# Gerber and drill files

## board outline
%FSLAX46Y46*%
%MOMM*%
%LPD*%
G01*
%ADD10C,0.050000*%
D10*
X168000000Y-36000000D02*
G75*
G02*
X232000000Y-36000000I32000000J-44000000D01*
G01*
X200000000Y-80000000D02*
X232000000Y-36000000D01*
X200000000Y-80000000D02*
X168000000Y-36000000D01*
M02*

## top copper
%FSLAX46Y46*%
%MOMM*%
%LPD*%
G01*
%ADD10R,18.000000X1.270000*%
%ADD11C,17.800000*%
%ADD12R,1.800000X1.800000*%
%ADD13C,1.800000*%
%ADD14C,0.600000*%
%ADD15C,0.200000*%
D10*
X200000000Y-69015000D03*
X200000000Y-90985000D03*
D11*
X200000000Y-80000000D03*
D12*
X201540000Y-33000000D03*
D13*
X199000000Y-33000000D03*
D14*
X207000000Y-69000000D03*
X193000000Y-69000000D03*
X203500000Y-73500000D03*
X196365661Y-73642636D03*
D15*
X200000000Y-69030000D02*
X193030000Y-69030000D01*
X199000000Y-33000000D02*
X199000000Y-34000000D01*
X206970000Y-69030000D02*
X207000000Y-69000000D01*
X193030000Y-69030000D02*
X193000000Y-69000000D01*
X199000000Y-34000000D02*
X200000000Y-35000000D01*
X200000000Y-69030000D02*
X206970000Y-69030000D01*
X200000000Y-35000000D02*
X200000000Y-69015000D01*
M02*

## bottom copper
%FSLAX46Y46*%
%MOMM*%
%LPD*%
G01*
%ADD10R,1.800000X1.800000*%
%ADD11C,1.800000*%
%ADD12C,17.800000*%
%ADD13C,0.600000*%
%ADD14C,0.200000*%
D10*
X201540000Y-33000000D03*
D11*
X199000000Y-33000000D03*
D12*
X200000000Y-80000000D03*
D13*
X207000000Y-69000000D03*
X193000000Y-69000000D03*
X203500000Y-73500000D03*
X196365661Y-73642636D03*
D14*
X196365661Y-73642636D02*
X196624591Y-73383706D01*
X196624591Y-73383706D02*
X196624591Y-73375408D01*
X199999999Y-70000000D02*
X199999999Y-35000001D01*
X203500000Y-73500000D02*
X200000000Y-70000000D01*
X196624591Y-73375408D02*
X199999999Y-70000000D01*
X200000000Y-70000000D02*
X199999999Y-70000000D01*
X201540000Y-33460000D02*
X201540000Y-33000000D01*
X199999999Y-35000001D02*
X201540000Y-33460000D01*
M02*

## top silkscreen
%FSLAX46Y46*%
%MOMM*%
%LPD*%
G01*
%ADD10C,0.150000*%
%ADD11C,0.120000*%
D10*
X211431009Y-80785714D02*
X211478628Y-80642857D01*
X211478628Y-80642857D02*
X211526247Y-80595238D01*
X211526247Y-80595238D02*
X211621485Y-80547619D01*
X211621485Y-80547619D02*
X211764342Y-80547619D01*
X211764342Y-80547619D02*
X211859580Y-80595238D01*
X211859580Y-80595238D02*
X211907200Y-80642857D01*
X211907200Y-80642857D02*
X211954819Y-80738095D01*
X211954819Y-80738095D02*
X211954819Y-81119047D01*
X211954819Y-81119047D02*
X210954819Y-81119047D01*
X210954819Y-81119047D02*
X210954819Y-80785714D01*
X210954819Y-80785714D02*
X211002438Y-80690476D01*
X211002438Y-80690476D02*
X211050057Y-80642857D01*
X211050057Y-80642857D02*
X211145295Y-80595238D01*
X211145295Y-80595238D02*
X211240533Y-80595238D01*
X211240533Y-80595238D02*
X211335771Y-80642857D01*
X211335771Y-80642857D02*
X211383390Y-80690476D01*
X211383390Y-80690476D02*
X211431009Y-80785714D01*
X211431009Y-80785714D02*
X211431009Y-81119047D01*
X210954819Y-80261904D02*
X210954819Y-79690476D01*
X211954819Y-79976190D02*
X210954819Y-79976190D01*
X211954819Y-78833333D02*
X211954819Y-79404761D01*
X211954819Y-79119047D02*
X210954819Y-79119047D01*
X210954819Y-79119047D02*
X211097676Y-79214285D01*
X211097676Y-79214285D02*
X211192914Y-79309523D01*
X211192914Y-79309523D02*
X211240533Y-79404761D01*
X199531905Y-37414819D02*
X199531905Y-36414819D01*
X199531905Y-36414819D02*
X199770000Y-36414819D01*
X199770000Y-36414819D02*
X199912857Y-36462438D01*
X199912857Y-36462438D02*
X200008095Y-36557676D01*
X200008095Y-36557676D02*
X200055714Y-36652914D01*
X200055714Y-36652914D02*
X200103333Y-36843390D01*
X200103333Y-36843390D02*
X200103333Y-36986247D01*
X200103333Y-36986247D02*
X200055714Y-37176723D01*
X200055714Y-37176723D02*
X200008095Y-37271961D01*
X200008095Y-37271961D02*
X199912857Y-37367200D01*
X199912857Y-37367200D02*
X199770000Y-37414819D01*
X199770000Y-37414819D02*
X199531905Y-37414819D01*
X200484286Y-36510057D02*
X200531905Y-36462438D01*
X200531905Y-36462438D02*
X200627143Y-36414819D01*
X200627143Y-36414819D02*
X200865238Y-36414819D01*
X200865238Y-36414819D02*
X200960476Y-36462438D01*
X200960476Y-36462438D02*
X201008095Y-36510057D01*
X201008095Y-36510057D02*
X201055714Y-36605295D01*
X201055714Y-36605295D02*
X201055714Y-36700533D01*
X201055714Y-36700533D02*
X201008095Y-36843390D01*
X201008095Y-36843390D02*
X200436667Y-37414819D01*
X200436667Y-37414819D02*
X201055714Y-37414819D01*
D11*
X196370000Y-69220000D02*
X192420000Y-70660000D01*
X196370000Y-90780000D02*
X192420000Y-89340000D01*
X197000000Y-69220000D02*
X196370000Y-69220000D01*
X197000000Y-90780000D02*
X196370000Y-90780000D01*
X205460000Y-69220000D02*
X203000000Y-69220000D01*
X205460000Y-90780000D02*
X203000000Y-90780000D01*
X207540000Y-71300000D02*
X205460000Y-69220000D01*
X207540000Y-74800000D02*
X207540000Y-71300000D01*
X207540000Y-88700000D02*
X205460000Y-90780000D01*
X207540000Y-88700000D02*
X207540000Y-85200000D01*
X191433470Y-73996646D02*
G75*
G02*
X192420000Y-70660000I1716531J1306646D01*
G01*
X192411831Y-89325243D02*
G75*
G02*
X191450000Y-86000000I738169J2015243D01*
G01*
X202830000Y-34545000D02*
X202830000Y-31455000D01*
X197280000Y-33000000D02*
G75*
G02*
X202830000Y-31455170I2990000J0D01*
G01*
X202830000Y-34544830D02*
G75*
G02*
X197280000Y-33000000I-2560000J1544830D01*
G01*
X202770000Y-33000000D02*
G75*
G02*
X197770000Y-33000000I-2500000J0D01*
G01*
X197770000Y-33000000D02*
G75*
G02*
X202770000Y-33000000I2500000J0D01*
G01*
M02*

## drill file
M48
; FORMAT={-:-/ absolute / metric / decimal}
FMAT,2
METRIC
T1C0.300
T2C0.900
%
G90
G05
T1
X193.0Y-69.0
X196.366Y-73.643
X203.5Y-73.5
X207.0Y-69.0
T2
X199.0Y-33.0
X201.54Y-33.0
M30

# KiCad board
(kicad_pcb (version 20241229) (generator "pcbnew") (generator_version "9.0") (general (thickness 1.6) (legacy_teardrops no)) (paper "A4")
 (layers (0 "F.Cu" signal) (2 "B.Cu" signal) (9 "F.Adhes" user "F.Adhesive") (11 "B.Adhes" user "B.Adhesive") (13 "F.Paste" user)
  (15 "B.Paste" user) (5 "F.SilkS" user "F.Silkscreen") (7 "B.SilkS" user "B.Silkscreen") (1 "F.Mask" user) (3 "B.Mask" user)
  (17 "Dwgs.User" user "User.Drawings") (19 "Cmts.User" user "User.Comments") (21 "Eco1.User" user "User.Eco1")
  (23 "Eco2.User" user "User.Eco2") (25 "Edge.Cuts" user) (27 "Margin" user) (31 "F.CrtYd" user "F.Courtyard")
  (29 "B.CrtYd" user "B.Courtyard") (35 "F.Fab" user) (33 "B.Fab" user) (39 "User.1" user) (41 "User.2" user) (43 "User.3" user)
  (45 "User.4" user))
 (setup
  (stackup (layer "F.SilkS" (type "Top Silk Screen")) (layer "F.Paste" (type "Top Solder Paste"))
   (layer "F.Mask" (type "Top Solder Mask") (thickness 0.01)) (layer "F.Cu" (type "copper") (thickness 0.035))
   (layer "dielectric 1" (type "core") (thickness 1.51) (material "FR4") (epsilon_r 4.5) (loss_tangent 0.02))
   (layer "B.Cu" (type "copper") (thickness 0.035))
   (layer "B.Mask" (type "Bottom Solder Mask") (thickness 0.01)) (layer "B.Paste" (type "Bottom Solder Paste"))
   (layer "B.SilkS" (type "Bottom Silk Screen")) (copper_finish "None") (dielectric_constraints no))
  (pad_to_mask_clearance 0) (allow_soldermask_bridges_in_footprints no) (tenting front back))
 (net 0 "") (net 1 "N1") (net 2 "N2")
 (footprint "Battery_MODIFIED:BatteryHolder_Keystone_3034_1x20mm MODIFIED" (layer "F.Cu") (at 200 80 -90)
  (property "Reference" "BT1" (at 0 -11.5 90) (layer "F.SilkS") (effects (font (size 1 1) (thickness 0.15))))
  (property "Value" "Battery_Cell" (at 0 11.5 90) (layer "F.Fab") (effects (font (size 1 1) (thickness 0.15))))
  (fp_line (start -10.78 3.63) (end -9.34 7.58) (stroke (width 0.12) (type solid)) (layer "F.SilkS"))
  (fp_line (start 10.78 3.63) (end 9.34 7.58) (stroke (width 0.12) (type solid)) (layer "F.SilkS"))
  (fp_line (start -10.78 3) (end -10.78 3.63) (stroke (width 0.12) (type solid)) (layer "F.SilkS"))
  (fp_line (start 10.78 3) (end 10.78 3.63) (stroke (width 0.12) (type solid)) (layer "F.SilkS"))
  (fp_line (start -10.78 -5.46) (end -10.78 -3) (stroke (width 0.12) (type solid)) (layer "F.SilkS"))
  (fp_line (start 10.78 -5.46) (end 10.78 -3) (stroke (width 0.12) (type solid)) (layer "F.SilkS"))
  (fp_line (start -8.7 -7.54) (end -10.78 -5.46) (stroke (width 0.12) (type solid)) (layer "F.SilkS"))
  (fp_line (start -5.2 -7.54) (end -8.7 -7.54) (stroke (width 0.12) (type solid)) (layer "F.SilkS"))
  (fp_line (start 8.7 -7.54) (end 10.78 -5.46) (stroke (width 0.12) (type solid)) (layer "F.SilkS"))
  (fp_line (start 8.7 -7.54) (end 5.2 -7.54) (stroke (width 0.12) (type solid)) (layer "F.SilkS"))
  (fp_arc (start -6.003354 8.56653) (mid -7.921654 8.918738) (end -9.34 7.58) (stroke (width 0.12) (type solid)) (layer "F.SilkS"))
  (fp_arc (start 9.325243 7.588169) (mid 7.90634 8.911668) (end 6 8.55) (stroke (width 0.12) (type solid)) (layer "F.SilkS"))
  (pad "1" smd rect (at -10.985 0 270) (size 1.27 18) (layers "F.Cu" "F.Mask" "F.Paste") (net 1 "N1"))
  (pad "1" smd rect (at 10.985 0 270) (size 1.27 18) (layers "F.Cu" "F.Mask" "F.Paste") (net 1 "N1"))
  (pad "2" smd circle (at 0 0 270) (size 17.8 17.8) (layers "F.Cu" "F.Mask") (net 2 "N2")))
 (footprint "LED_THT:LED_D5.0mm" (layer "F.Cu") (at 201.54 33 180)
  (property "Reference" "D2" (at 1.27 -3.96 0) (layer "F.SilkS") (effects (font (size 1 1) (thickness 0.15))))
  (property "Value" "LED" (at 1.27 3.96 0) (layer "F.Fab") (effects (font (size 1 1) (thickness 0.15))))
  (fp_line (start -1.29 -1.545) (end -1.29 1.545) (stroke (width 0.12) (type solid)) (layer "F.SilkS"))
  (fp_arc (start 4.26 0) (mid 2.071779 2.880495) (end -1.29 1.54483) (stroke (width 0.12) (type solid)) (layer "F.SilkS"))
  (fp_arc (start -1.29 -1.54483) (mid 2.071779 -2.880495) (end 4.26 0) (stroke (width 0.12) (type solid)) (layer "F.SilkS"))
  (fp_circle (center 1.27 0) (end 3.77 0) (stroke (width 0.12) (type solid)) (fill no) (layer "F.SilkS"))
  (pad "1" thru_hole rect (at 0 0 180) (size 1.8 1.8) (drill 0.9) (layers "*.Cu" "*.Mask") (remove_unused_layers no) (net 2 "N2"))
  (pad "2" thru_hole circle (at 2.54 0 180) (size 1.8 1.8) (drill 0.9) (layers "*.Cu" "*.Mask") (remove_unused_layers no) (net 1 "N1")))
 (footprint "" (layer "B.Cu") (at 200 80 180)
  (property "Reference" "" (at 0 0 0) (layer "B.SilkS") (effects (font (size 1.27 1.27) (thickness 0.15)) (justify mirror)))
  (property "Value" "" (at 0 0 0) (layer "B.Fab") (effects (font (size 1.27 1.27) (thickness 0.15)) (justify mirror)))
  (pad "2" smd circle (at 0 0 90) (size 17.8 17.8) (layers "B.Cu" "B.Mask") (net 2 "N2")))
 (gr_arc (start 168 36) (mid 200 25.594118) (end 232 36) (stroke (width 0.05) (type default)) (layer "Edge.Cuts"))
 (gr_line (start 200 80) (end 232 36) (stroke (width 0.05) (type default)) (layer "Edge.Cuts"))
 (gr_line (start 200 80) (end 168 36) (stroke (width 0.05) (type default)) (layer "Edge.Cuts"))
 (segment (start 200 69.03) (end 193.03 69.03) (width 0.2) (layer "F.Cu") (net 1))
 (segment (start 199 33) (end 199 34) (width 0.2) (layer "F.Cu") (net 1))
 (segment (start 206.97 69.03) (end 207 69) (width 0.2) (layer "F.Cu") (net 1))
 (segment (start 193.03 69.03) (end 193 69) (width 0.2) (layer "F.Cu") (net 1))
 (segment (start 199 34) (end 200 35) (width 0.2) (layer "F.Cu") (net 1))
 (segment (start 200 69.03) (end 206.97 69.03) (width 0.2) (layer "F.Cu") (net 1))
 (segment (start 200 35) (end 200 69.015) (width 0.2) (layer "F.Cu") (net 1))
 (via (at 207 69) (size 0.6) (drill 0.3) (layers "F.Cu" "B.Cu") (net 1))
 (via (at 193 69) (size 0.6) (drill 0.3) (layers "F.Cu" "B.Cu") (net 1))
 (via (at 203.5 73.5) (size 0.6) (drill 0.3) (layers "F.Cu" "B.Cu") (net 2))
 (via (at 196.365661 73.642636) (size 0.6) (drill 0.3) (layers "F.Cu" "B.Cu") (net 2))
 (segment (start 196.365661 73.642636) (end 196.624591 73.383706) (width 0.2) (layer "B.Cu") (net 2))
 (segment (start 196.624591 73.383706) (end 196.624591 73.375408) (width 0.2) (layer "B.Cu") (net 2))
 (segment (start 199.999999 70) (end 199.999999 35.000001) (width 0.2) (layer "B.Cu") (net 2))
 (segment (start 203.5 73.5) (end 200 70) (width 0.2) (layer "B.Cu") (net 2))
 (segment (start 196.624591 73.375408) (end 199.999999 70) (width 0.2) (layer "B.Cu") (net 2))
 (segment (start 200 70) (end 199.999999 70) (width 0.2) (layer "B.Cu") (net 2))
 (segment (start 201.54 33.46) (end 201.54 33) (width 0.2) (layer "B.Cu") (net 2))
 (segment (start 199.999999 35.000001) (end 201.54 33.46) (width 0.2) (layer "B.Cu") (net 2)))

